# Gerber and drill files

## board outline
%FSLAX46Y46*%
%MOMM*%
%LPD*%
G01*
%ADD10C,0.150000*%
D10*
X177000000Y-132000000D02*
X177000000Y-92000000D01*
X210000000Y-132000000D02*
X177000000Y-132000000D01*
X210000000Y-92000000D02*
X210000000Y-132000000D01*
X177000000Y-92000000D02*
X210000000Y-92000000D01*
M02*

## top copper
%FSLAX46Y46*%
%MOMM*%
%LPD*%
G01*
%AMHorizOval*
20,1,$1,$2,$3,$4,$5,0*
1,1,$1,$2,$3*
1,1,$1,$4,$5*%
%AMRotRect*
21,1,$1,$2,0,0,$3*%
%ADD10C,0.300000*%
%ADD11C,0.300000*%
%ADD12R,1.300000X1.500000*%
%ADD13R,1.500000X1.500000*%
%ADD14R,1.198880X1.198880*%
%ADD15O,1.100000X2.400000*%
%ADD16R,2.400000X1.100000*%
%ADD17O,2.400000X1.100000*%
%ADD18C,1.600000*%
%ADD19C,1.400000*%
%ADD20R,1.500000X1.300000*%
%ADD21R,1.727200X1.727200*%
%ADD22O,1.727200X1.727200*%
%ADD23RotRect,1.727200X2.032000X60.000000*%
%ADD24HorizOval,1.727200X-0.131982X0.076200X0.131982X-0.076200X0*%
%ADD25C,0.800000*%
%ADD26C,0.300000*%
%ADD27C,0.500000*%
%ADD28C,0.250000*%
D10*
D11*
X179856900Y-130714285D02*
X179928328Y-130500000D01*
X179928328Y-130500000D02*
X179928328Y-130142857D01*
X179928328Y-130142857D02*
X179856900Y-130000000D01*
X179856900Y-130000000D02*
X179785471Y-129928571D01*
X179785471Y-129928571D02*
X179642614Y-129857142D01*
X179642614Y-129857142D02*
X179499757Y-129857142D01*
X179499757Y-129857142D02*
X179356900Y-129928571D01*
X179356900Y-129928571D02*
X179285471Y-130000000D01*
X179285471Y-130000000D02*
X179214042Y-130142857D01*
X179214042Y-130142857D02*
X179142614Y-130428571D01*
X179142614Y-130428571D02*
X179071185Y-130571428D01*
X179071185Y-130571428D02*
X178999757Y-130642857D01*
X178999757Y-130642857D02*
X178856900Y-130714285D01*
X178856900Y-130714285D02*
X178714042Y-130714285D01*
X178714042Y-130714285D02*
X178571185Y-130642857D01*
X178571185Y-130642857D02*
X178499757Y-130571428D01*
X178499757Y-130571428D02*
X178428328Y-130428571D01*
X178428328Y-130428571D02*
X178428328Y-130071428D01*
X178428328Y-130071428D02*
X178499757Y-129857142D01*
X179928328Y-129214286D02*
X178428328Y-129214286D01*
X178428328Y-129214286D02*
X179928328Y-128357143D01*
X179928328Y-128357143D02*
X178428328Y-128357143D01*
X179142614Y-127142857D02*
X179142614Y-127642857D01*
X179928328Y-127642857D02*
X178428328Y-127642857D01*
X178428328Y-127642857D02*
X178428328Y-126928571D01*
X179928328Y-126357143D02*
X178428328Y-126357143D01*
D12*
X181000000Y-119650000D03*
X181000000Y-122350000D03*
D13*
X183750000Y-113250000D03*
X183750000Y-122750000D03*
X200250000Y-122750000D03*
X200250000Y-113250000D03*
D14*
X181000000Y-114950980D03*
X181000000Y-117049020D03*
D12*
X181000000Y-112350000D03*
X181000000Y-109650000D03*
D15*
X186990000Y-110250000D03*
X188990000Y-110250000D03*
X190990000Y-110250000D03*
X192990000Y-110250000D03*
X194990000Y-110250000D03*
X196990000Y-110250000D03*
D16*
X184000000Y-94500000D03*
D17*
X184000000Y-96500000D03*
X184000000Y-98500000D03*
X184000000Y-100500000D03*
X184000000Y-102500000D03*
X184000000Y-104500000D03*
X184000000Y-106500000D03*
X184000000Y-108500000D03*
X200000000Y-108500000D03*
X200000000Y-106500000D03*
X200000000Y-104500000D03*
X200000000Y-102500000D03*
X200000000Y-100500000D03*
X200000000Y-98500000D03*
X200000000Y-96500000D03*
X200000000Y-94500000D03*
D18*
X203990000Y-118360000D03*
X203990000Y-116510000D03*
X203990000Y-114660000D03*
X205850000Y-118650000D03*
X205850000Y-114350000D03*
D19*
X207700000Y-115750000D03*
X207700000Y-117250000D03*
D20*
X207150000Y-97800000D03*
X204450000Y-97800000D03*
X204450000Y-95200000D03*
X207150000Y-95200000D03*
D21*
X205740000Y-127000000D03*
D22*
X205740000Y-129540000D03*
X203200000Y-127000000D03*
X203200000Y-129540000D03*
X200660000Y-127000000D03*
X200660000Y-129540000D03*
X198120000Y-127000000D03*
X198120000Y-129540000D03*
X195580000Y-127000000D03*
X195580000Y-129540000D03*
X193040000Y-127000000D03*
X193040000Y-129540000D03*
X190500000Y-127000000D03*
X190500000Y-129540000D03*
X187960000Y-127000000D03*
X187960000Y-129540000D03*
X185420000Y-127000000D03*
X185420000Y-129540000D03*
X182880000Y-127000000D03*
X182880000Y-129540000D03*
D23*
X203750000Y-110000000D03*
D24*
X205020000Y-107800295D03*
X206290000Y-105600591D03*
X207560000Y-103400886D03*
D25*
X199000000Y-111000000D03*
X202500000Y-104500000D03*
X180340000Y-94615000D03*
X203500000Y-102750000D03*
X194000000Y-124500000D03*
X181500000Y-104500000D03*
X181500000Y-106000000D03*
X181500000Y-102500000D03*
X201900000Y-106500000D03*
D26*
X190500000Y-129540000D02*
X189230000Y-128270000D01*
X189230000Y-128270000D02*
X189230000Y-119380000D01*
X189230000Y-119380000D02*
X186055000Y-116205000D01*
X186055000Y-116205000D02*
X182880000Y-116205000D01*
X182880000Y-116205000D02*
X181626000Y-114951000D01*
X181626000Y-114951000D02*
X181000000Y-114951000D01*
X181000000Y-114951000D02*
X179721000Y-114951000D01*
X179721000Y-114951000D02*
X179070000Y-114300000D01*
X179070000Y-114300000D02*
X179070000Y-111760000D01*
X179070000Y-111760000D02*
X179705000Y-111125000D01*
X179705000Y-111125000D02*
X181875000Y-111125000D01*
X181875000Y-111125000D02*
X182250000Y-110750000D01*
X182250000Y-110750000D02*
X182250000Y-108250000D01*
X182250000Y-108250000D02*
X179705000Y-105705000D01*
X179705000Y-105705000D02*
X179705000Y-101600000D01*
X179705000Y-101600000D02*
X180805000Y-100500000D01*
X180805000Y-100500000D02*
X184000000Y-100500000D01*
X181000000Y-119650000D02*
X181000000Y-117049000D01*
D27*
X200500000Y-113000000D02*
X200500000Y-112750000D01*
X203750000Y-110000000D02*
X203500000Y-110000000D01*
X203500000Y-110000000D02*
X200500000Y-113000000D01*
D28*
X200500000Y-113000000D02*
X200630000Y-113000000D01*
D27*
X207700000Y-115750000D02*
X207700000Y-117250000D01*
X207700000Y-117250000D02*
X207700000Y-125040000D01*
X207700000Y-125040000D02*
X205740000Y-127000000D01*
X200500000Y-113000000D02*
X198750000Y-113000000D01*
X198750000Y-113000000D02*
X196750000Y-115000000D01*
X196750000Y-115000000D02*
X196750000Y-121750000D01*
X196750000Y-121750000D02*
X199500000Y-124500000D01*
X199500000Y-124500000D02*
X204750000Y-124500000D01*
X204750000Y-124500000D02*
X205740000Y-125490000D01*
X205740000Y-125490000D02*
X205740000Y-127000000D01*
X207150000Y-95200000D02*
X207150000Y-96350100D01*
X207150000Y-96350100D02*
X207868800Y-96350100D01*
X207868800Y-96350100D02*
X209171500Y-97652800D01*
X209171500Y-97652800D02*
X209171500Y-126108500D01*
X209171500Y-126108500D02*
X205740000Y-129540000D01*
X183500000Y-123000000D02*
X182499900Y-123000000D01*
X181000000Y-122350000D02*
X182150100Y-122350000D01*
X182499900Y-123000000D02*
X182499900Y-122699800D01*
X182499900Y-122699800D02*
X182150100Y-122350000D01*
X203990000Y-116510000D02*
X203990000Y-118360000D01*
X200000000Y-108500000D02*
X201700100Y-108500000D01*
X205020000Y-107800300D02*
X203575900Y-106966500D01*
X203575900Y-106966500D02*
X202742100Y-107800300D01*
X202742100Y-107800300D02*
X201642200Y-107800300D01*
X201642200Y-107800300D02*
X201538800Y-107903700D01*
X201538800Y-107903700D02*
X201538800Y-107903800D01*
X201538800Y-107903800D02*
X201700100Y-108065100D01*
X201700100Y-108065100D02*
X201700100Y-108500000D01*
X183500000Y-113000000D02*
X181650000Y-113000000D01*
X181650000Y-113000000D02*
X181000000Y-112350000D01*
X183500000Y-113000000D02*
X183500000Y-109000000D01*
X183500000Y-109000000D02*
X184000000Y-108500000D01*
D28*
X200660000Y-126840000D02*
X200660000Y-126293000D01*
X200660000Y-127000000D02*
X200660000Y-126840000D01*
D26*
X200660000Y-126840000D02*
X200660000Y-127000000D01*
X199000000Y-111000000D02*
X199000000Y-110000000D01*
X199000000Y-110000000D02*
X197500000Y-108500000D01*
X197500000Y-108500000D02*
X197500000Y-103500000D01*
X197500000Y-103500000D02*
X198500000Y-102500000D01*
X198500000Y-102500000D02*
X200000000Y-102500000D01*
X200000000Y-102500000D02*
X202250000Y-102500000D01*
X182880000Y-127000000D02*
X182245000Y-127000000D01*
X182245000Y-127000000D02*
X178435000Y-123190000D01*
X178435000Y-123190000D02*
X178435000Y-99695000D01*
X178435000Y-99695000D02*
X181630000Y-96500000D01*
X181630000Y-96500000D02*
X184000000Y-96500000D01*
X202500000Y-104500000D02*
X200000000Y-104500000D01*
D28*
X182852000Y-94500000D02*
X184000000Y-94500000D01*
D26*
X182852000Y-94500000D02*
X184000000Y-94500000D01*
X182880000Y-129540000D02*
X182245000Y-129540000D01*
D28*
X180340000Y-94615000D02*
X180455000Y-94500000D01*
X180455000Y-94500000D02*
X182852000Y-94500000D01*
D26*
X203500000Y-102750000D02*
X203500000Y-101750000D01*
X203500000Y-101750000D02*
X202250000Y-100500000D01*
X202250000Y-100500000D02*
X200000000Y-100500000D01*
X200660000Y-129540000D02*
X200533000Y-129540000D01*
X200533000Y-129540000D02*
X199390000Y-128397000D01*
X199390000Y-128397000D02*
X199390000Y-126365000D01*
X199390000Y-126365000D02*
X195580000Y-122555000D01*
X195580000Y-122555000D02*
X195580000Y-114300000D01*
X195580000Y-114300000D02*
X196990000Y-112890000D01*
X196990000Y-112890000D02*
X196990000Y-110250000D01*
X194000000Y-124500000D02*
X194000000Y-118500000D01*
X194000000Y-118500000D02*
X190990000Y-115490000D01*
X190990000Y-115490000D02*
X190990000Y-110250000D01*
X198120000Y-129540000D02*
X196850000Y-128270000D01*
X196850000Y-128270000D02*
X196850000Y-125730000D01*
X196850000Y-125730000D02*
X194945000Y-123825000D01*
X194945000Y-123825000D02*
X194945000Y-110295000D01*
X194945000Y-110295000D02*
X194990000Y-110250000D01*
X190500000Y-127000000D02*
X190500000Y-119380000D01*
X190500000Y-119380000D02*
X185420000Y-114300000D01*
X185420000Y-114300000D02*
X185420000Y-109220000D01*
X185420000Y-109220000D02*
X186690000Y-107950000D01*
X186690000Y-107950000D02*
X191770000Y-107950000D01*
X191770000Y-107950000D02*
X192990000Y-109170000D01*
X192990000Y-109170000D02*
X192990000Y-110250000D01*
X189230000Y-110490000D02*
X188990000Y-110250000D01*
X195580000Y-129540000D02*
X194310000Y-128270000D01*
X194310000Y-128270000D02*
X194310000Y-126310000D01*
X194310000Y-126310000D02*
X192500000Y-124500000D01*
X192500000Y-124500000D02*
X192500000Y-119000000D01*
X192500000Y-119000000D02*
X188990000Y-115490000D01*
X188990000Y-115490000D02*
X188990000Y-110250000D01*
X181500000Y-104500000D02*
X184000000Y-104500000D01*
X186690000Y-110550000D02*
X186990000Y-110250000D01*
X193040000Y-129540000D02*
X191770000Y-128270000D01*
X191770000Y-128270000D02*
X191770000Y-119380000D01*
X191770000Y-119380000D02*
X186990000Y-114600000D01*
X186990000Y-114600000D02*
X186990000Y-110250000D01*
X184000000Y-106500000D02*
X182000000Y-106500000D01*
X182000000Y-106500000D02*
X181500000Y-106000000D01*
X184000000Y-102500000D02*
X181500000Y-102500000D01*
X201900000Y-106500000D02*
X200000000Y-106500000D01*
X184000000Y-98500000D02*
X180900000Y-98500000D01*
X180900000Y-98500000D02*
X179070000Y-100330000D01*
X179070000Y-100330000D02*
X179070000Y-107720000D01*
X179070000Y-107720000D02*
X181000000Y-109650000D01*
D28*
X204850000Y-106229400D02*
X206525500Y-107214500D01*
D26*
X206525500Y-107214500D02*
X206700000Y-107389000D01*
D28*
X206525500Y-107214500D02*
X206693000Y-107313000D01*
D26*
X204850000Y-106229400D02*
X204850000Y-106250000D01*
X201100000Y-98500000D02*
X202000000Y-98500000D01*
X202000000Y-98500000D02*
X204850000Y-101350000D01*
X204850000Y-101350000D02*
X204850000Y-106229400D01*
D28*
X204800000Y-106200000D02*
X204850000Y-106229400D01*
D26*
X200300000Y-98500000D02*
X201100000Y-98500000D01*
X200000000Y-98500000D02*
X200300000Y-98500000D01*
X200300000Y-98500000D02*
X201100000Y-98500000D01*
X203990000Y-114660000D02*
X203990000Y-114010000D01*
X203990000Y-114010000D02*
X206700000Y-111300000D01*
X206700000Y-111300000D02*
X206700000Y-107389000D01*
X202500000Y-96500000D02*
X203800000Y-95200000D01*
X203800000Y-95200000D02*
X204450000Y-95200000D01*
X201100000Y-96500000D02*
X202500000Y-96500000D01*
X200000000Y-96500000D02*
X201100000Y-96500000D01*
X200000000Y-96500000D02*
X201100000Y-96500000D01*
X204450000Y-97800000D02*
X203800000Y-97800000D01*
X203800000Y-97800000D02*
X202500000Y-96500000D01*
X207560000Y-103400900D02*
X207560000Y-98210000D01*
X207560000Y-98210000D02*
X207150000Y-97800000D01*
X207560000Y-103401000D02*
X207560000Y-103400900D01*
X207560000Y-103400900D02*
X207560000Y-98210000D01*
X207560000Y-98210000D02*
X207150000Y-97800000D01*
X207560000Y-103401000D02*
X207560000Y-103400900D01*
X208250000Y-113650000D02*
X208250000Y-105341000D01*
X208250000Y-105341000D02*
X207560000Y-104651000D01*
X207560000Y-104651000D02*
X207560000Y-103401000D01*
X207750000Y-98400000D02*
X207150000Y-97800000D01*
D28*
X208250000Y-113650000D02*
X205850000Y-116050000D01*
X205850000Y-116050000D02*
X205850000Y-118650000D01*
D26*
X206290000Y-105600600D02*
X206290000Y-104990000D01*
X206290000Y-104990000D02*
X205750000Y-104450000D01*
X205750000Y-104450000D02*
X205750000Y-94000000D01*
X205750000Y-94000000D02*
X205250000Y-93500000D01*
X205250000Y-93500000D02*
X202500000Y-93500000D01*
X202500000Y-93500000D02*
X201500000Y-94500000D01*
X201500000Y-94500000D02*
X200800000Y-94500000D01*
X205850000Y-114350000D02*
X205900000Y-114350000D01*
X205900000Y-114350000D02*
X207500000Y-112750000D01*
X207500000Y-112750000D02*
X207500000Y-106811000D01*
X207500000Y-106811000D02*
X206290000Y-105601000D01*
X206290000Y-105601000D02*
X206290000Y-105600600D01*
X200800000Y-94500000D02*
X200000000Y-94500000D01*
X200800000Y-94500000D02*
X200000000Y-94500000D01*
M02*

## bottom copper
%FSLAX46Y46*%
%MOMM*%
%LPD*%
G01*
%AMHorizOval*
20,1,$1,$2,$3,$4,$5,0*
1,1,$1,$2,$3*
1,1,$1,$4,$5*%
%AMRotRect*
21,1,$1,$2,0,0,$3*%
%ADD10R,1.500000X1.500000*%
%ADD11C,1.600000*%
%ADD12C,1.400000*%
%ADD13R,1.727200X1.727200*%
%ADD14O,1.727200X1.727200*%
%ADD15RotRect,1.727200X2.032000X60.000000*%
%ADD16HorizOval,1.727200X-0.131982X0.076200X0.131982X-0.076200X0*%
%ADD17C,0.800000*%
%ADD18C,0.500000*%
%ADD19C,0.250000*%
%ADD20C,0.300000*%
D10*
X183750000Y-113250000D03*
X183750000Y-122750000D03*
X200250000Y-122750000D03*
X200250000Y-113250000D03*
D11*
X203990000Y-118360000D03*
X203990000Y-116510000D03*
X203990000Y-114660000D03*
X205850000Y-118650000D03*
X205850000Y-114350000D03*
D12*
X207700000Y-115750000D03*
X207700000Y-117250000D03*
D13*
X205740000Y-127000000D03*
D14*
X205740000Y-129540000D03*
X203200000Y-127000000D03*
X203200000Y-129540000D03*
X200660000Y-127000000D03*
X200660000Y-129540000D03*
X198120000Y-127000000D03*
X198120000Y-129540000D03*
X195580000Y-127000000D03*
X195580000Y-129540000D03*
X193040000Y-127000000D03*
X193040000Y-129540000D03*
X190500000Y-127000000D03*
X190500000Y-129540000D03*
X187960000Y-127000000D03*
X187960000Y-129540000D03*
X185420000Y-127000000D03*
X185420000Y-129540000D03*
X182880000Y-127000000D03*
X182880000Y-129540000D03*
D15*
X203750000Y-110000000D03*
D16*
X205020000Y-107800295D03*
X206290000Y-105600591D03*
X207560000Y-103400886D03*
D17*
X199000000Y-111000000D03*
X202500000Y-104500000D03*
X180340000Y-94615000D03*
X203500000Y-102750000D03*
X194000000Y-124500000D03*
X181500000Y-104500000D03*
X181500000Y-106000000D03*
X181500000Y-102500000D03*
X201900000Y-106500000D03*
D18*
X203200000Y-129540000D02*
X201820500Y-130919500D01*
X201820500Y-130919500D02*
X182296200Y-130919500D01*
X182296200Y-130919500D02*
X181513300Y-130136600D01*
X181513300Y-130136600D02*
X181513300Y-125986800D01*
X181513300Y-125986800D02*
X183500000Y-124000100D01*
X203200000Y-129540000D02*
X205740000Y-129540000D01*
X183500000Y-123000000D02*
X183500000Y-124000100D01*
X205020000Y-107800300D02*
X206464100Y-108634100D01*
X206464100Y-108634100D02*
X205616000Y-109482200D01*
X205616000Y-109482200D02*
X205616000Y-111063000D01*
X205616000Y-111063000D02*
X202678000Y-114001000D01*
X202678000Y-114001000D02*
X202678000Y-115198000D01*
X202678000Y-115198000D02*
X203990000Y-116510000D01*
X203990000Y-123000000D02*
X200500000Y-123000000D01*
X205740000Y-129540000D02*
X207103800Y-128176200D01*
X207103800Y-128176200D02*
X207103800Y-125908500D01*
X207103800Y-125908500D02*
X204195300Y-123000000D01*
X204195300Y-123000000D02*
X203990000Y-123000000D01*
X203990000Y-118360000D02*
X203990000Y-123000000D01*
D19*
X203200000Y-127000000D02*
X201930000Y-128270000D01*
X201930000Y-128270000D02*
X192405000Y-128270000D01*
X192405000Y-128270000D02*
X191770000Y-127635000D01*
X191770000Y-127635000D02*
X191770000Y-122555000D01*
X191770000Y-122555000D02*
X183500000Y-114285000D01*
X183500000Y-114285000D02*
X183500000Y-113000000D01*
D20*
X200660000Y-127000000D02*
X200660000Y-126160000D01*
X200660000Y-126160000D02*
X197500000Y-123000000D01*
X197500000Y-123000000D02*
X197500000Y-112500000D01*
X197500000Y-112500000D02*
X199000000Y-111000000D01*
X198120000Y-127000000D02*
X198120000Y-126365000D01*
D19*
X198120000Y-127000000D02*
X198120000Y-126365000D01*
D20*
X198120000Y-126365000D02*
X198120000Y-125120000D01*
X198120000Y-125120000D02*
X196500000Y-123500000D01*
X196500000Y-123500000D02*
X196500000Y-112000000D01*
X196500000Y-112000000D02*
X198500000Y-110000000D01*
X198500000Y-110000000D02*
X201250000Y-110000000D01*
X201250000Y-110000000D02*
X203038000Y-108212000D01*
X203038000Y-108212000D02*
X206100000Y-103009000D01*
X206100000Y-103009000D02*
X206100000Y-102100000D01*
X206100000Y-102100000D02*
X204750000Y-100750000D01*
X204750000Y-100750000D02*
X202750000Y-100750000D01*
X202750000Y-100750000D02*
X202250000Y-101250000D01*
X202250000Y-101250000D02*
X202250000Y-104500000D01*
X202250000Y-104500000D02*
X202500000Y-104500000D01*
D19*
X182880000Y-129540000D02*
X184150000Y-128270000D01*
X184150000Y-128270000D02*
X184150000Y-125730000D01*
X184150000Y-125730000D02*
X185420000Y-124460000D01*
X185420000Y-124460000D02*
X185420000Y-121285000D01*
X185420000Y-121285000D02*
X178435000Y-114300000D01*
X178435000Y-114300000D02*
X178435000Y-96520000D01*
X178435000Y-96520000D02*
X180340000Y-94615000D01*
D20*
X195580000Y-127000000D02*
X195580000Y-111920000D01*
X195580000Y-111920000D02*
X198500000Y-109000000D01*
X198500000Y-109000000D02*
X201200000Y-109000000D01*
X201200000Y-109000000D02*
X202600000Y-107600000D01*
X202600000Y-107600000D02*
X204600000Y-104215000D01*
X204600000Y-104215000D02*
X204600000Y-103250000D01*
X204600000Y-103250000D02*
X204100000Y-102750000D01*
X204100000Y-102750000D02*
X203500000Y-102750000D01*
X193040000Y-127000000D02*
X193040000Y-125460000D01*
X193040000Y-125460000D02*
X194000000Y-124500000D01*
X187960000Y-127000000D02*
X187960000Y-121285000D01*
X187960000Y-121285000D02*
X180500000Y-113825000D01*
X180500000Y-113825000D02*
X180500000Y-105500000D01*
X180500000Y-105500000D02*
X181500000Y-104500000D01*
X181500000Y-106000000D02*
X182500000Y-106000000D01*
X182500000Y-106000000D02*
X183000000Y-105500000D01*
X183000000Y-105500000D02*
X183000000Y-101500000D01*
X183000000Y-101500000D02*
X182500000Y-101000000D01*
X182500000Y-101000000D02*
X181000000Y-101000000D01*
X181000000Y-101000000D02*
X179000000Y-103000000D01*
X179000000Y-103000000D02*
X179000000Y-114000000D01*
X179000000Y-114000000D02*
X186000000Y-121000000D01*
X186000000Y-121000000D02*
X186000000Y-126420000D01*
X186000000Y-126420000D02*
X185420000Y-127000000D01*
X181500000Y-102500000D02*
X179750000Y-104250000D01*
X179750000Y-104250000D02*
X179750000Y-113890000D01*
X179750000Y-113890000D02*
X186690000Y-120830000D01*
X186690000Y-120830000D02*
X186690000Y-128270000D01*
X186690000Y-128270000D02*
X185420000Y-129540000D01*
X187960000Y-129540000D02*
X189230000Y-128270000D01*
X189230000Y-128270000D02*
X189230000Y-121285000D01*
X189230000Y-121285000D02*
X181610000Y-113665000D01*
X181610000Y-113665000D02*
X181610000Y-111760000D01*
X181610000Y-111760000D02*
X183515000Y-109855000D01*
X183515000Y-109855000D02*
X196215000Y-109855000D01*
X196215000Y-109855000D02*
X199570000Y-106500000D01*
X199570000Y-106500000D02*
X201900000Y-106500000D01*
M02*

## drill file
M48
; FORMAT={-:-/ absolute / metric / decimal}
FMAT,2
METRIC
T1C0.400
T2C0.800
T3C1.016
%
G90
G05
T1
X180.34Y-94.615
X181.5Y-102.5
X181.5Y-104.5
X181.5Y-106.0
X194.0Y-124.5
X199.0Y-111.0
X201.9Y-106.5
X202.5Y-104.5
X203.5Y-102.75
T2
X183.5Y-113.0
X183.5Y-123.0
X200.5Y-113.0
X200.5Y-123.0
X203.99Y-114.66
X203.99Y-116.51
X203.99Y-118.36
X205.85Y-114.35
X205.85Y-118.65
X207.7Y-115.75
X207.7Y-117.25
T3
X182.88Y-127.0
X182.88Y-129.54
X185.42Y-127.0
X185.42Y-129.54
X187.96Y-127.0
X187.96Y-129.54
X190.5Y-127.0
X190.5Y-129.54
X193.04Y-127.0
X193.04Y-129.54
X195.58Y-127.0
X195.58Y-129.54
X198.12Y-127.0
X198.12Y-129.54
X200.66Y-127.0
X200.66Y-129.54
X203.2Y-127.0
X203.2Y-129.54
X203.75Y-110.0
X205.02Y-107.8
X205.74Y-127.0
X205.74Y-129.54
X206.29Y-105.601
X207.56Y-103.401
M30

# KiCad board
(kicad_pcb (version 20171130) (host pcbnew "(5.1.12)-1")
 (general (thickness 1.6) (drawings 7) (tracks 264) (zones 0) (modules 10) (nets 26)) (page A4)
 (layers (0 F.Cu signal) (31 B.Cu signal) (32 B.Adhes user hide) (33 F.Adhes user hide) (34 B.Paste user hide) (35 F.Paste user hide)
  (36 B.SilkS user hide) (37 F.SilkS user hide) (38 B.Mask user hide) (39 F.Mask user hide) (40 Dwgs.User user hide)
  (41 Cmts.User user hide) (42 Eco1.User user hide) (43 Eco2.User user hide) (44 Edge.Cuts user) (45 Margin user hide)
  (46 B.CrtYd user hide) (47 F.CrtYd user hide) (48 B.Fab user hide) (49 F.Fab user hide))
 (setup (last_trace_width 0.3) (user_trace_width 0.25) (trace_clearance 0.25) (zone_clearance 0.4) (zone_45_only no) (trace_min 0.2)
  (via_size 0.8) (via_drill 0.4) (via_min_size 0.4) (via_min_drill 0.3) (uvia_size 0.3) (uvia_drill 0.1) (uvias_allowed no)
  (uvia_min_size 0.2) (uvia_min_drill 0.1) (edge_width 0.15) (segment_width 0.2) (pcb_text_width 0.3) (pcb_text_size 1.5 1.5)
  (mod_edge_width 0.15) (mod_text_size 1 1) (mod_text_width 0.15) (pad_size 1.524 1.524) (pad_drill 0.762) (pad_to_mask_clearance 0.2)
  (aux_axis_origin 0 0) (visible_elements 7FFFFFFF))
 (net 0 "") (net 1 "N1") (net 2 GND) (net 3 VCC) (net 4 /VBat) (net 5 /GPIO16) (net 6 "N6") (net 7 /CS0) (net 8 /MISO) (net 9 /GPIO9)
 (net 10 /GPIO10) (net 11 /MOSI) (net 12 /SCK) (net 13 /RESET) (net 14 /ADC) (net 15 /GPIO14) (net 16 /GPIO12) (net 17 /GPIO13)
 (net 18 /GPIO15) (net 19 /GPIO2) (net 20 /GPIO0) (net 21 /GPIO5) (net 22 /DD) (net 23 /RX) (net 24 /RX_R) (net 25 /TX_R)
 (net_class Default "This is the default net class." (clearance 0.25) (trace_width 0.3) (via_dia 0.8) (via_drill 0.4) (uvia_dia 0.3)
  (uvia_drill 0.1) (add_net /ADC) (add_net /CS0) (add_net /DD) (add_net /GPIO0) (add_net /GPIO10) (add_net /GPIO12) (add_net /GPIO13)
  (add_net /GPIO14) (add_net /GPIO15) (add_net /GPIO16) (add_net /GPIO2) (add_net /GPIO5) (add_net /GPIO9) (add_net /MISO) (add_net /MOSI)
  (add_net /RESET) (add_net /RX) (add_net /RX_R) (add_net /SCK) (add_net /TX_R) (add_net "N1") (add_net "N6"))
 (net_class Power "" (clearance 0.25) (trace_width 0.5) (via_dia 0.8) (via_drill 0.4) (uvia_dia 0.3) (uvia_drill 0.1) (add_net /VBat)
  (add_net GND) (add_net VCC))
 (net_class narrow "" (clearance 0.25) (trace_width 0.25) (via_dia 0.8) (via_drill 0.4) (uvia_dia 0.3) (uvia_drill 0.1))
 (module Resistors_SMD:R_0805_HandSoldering (layer F.Cu) (at 181 121 270)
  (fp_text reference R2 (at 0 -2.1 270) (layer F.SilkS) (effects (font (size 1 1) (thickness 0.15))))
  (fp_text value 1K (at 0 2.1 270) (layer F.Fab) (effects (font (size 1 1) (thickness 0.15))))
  (pad 1 smd rect (at -1.35 0 270) (size 1.5 1.3) (layers F.Cu F.Paste F.Mask) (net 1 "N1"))
  (pad 2 smd rect (at 1.35 0 270) (size 1.5 1.3) (layers F.Cu F.Paste F.Mask) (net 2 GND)))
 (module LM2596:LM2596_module (layer F.Cu) (at 192 118)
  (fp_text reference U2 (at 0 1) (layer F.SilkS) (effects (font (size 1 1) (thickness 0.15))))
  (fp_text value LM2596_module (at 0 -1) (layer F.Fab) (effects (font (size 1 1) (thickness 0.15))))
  (pad 1 thru_hole rect (at -8.5 -5) (size 1.5 1.5) (drill 0.8 (offset 0.25 0.25)) (layers *.Cu *.Mask F.SilkS) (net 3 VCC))
  (pad 2 thru_hole rect (at -8.5 5) (size 1.5 1.5) (drill 0.8 (offset 0.25 -0.25)) (layers *.Cu *.Mask F.SilkS) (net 2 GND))
  (pad 3 thru_hole rect (at 8.5 5) (size 1.5 1.5) (drill 0.8 (offset -0.25 -0.25)) (layers *.Cu *.Mask F.SilkS) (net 2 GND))
  (pad 4 thru_hole rect (at 8.5 -5) (size 1.5 1.5) (drill 0.8 (offset -0.25 0.25)) (layers *.Cu *.Mask F.SilkS) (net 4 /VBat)))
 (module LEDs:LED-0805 (layer F.Cu) (at 181 116 90)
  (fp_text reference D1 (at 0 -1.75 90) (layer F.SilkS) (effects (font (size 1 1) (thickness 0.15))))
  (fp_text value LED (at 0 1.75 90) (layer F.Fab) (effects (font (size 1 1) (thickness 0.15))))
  (pad 2 smd rect (at 1.04902 0 270) (size 1.19888 1.19888) (layers F.Cu F.Paste F.Mask) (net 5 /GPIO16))
  (pad 1 smd rect (at -1.04902 0 270) (size 1.19888 1.19888) (layers F.Cu F.Paste F.Mask) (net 1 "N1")))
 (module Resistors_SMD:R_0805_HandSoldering (layer F.Cu) (at 181 111 90)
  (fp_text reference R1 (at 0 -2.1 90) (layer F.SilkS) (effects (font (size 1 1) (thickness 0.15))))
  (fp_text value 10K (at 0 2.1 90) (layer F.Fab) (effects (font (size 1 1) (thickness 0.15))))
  (pad 1 smd rect (at -1.35 0 90) (size 1.5 1.3) (layers F.Cu F.Paste F.Mask) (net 3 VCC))
  (pad 2 smd rect (at 1.35 0 90) (size 1.5 1.3) (layers F.Cu F.Paste F.Mask) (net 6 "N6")))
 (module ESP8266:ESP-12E (layer F.Cu) (at 184 94.5)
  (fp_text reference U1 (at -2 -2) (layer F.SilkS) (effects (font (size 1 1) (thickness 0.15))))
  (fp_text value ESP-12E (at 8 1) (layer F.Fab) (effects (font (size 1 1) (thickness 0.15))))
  (pad 9 smd oval (at 2.99 15.75 90) (size 2.4 1.1) (layers F.Cu F.Paste F.Mask) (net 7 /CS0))
  (pad 10 smd oval (at 4.99 15.75 90) (size 2.4 1.1) (layers F.Cu F.Paste F.Mask) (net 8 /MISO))
  (pad 11 smd oval (at 6.99 15.75 90) (size 2.4 1.1) (layers F.Cu F.Paste F.Mask) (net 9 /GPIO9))
  (pad 12 smd oval (at 8.99 15.75 90) (size 2.4 1.1) (layers F.Cu F.Paste F.Mask) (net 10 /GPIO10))
  (pad 13 smd oval (at 10.99 15.75 90) (size 2.4 1.1) (layers F.Cu F.Paste F.Mask) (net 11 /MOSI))
  (pad 14 smd oval (at 12.99 15.75 90) (size 2.4 1.1) (layers F.Cu F.Paste F.Mask) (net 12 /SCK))
  (pad 1 smd rect (at 0 0) (size 2.4 1.1) (layers F.Cu F.Paste F.Mask) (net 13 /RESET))
  (pad 2 smd oval (at 0 2) (size 2.4 1.1) (layers F.Cu F.Paste F.Mask) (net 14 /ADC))
  (pad 3 smd oval (at 0 4) (size 2.4 1.1) (layers F.Cu F.Paste F.Mask) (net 6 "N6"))
  (pad 4 smd oval (at 0 6) (size 2.4 1.1) (layers F.Cu F.Paste F.Mask) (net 5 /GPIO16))
  (pad 5 smd oval (at 0 8) (size 2.4 1.1) (layers F.Cu F.Paste F.Mask) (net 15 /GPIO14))
  (pad 6 smd oval (at 0 10) (size 2.4 1.1) (layers F.Cu F.Paste F.Mask) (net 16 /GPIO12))
  (pad 7 smd oval (at 0 12) (size 2.4 1.1) (layers F.Cu F.Paste F.Mask) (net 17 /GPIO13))
  (pad 8 smd oval (at 0 14) (size 2.4 1.1) (layers F.Cu F.Paste F.Mask) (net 3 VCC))
  (pad 15 smd oval (at 16 14) (size 2.4 1.1) (layers F.Cu F.Paste F.Mask) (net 2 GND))
  (pad 16 smd oval (at 16 12) (size 2.4 1.1) (layers F.Cu F.Paste F.Mask) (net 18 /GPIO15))
  (pad 17 smd oval (at 16 10) (size 2.4 1.1) (layers F.Cu F.Paste F.Mask) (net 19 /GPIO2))
  (pad 18 smd oval (at 16 8) (size 2.4 1.1) (layers F.Cu F.Paste F.Mask) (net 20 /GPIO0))
  (pad 19 smd oval (at 16 6) (size 2.4 1.1) (layers F.Cu F.Paste F.Mask) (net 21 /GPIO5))
  (pad 20 smd oval (at 16 4) (size 2.4 1.1) (layers F.Cu F.Paste F.Mask) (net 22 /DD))
  (pad 21 smd oval (at 16 2) (size 2.4 1.1) (layers F.Cu F.Paste F.Mask) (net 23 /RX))
  (pad 22 smd oval (at 16 0) (size 2.4 1.1) (layers F.Cu F.Paste F.Mask) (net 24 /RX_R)))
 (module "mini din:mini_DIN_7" (layer F.Cu) (at 213.5 116.5 90)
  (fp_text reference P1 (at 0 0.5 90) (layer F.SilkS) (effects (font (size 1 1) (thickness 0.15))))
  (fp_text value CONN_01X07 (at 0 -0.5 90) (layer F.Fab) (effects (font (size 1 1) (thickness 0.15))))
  (pad 7 thru_hole circle (at -1.86 -9.51 90) (size 1.6 1.6) (drill 0.8) (layers *.Cu *.Mask F.SilkS) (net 2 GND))
  (pad 6 thru_hole circle (at -0.01 -9.51 90) (size 1.6 1.6) (drill 0.8) (layers *.Cu *.Mask F.SilkS) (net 2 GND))
  (pad 5 thru_hole circle (at 1.84 -9.51 90) (size 1.6 1.6) (drill 0.8) (layers *.Cu *.Mask F.SilkS) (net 22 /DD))
  (pad 4 thru_hole circle (at -2.15 -7.65 90) (size 1.6 1.6) (drill 0.8) (layers *.Cu *.Mask F.SilkS) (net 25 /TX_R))
  (pad 3 thru_hole circle (at 2.15 -7.65 90) (size 1.6 1.6) (drill 0.8) (layers *.Cu *.Mask F.SilkS) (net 24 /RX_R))
  (pad 1 thru_hole circle (at 0.75 -5.8 90) (size 1.4 1.4) (drill 0.8) (layers *.Cu *.Mask F.SilkS) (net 4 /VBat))
  (pad 2 thru_hole circle (at -0.75 -5.8 90) (size 1.4 1.4) (drill 0.8) (layers *.Cu *.Mask F.SilkS) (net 4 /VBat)))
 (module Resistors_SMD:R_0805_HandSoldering (layer F.Cu) (at 205.8 97.8 180)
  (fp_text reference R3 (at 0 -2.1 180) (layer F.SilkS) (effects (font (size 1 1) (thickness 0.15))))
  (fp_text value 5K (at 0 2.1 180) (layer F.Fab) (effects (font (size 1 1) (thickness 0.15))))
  (pad 1 smd rect (at -1.35 0 180) (size 1.5 1.3) (layers F.Cu F.Paste F.Mask) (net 25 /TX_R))
  (pad 2 smd rect (at 1.35 0 180) (size 1.5 1.3) (layers F.Cu F.Paste F.Mask) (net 23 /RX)))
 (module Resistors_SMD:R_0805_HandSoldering (layer F.Cu) (at 205.8 95.2)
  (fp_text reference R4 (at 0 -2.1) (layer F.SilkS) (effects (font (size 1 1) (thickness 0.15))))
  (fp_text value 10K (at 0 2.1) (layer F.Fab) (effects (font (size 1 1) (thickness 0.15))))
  (pad 1 smd rect (at -1.35 0) (size 1.5 1.3) (layers F.Cu F.Paste F.Mask) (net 23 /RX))
  (pad 2 smd rect (at 1.35 0) (size 1.5 1.3) (layers F.Cu F.Paste F.Mask) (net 2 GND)))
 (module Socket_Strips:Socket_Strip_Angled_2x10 (layer B.Cu) (at 205.74 127 180)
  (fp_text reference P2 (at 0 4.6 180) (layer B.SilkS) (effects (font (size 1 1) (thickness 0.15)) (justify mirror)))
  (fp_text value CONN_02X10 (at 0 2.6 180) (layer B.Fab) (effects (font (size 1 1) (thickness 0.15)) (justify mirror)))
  (pad 1 thru_hole rect (at 0 0 180) (size 1.7272 1.7272) (drill 1.016) (layers *.Cu *.Mask B.SilkS) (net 4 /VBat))
  (pad 2 thru_hole oval (at 0 -2.54 180) (size 1.7272 1.7272) (drill 1.016) (layers *.Cu *.Mask B.SilkS) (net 2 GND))
  (pad 3 thru_hole oval (at 2.54 0 180) (size 1.7272 1.7272) (drill 1.016) (layers *.Cu *.Mask B.SilkS) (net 3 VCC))
  (pad 4 thru_hole oval (at 2.54 -2.54 180) (size 1.7272 1.7272) (drill 1.016) (layers *.Cu *.Mask B.SilkS) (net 2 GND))
  (pad 5 thru_hole oval (at 5.08 0 180) (size 1.7272 1.7272) (drill 1.016) (layers *.Cu *.Mask B.SilkS) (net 20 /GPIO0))
  (pad 6 thru_hole oval (at 5.08 -2.54 180) (size 1.7272 1.7272) (drill 1.016) (layers *.Cu *.Mask B.SilkS) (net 12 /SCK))
  (pad 7 thru_hole oval (at 7.62 0 180) (size 1.7272 1.7272) (drill 1.016) (layers *.Cu *.Mask B.SilkS) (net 19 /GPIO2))
  (pad 8 thru_hole oval (at 7.62 -2.54 180) (size 1.7272 1.7272) (drill 1.016) (layers *.Cu *.Mask B.SilkS) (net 11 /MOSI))
  (pad 9 thru_hole oval (at 10.16 0 180) (size 1.7272 1.7272) (drill 1.016) (layers *.Cu *.Mask B.SilkS) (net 21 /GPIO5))
  (pad 10 thru_hole oval (at 10.16 -2.54 180) (size 1.7272 1.7272) (drill 1.016) (layers *.Cu *.Mask B.SilkS) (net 8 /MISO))
  (pad 11 thru_hole oval (at 12.7 0 180) (size 1.7272 1.7272) (drill 1.016) (layers *.Cu *.Mask B.SilkS) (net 9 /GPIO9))
  (pad 12 thru_hole oval (at 12.7 -2.54 180) (size 1.7272 1.7272) (drill 1.016) (layers *.Cu *.Mask B.SilkS) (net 7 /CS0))
  (pad 13 thru_hole oval (at 15.24 0 180) (size 1.7272 1.7272) (drill 1.016) (layers *.Cu *.Mask B.SilkS) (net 10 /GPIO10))
  (pad 14 thru_hole oval (at 15.24 -2.54 180) (size 1.7272 1.7272) (drill 1.016) (layers *.Cu *.Mask B.SilkS) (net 5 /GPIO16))
  (pad 15 thru_hole oval (at 17.78 0 180) (size 1.7272 1.7272) (drill 1.016) (layers *.Cu *.Mask B.SilkS) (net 16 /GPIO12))
  (pad 16 thru_hole oval (at 17.78 -2.54 180) (size 1.7272 1.7272) (drill 1.016) (layers *.Cu *.Mask B.SilkS) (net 18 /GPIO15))
  (pad 17 thru_hole oval (at 20.32 0 180) (size 1.7272 1.7272) (drill 1.016) (layers *.Cu *.Mask B.SilkS) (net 17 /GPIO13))
  (pad 18 thru_hole oval (at 20.32 -2.54 180) (size 1.7272 1.7272) (drill 1.016) (layers *.Cu *.Mask B.SilkS) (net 15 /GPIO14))
  (pad 19 thru_hole oval (at 22.86 0 180) (size 1.7272 1.7272) (drill 1.016) (layers *.Cu *.Mask B.SilkS) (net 14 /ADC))
  (pad 20 thru_hole oval (at 22.86 -2.54 180) (size 1.7272 1.7272) (drill 1.016) (layers *.Cu *.Mask B.SilkS) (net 13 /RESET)))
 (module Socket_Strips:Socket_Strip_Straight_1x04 (layer F.Cu) (at 203.75 110 60)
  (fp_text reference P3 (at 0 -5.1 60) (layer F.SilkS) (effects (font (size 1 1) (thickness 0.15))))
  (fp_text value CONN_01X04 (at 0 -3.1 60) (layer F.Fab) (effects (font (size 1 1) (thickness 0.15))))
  (pad 1 thru_hole rect (at 0 0 60) (size 1.7272 2.032) (drill 1.016) (layers *.Cu *.Mask F.SilkS) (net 4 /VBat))
  (pad 2 thru_hole oval (at 2.54 0 60) (size 1.7272 2.032) (drill 1.016) (layers *.Cu *.Mask F.SilkS) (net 2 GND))
  (pad 3 thru_hole oval (at 5.08 0 60) (size 1.7272 2.032) (drill 1.016) (layers *.Cu *.Mask F.SilkS) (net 24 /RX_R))
  (pad 4 thru_hole oval (at 7.62 0 60) (size 1.7272 2.032) (drill 1.016) (layers *.Cu *.Mask F.SilkS) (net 25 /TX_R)))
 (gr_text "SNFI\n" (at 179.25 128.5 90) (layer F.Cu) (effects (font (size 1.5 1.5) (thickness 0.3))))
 (gr_line (start 177 132) (end 177 92) (angle 90) (layer Edge.Cuts) (width 0.15))
 (gr_line (start 210 132) (end 177 132) (angle 90) (layer Edge.Cuts) (width 0.15))
 (gr_line (start 210 92) (end 210 132) (angle 90) (layer Edge.Cuts) (width 0.15))
 (gr_line (start 177 92) (end 210 92) (angle 90) (layer Edge.Cuts) (width 0.15))
 (segment (start 190.5 129.54) (end 189.23 128.27) (width 0.3) (layer F.Cu) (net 5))
 (segment (start 189.23 128.27) (end 189.23 119.38) (width 0.3) (layer F.Cu) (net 5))
 (segment (start 189.23 119.38) (end 186.055 116.205) (width 0.3) (layer F.Cu) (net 5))
 (segment (start 186.055 116.205) (end 182.88 116.205) (width 0.3) (layer F.Cu) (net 5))
 (segment (start 182.88 116.205) (end 181.626 114.951) (width 0.3) (layer F.Cu) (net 5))
 (segment (start 181.626 114.951) (end 181 114.951) (width 0.3) (layer F.Cu) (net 5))
 (segment (start 181 114.951) (end 179.721 114.951) (width 0.3) (layer F.Cu) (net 5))
 (segment (start 179.721 114.951) (end 179.07 114.3) (width 0.3) (layer F.Cu) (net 5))
 (segment (start 179.07 114.3) (end 179.07 111.76) (width 0.3) (layer F.Cu) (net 5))
 (segment (start 179.07 111.76) (end 179.705 111.125) (width 0.3) (layer F.Cu) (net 5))
 (segment (start 179.705 111.125) (end 181.875 111.125) (width 0.3) (layer F.Cu) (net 5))
 (segment (start 181.875 111.125) (end 182.25 110.75) (width 0.3) (layer F.Cu) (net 5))
 (segment (start 182.25 110.75) (end 182.25 108.25) (width 0.3) (layer F.Cu) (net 5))
 (segment (start 182.25 108.25) (end 179.705 105.705) (width 0.3) (layer F.Cu) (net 5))
 (segment (start 179.705 105.705) (end 179.705 101.6) (width 0.3) (layer F.Cu) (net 5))
 (segment (start 179.705 101.6) (end 180.805 100.5) (width 0.3) (layer F.Cu) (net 5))
 (segment (start 180.805 100.5) (end 184 100.5) (width 0.3) (layer F.Cu) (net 5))
 (segment (start 181 119.65) (end 181 117.049) (width 0.3) (layer F.Cu) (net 1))
 (segment (start 200.5 113) (end 200.5 112.75) (width 0.5) (layer F.Cu) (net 4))
 (segment (start 203.75 110) (end 203.5 110) (width 0.5) (layer F.Cu) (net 4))
 (segment (start 203.5 110) (end 200.5 113) (width 0.5) (layer F.Cu) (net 4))
 (segment (start 200.5 113) (end 200.63 113) (width 0.25) (layer F.Cu) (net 4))
 (segment (start 207.7 115.75) (end 207.7 117.25) (width 0.5) (layer F.Cu) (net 4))
 (segment (start 207.7 117.25) (end 207.7 125.04) (width 0.5) (layer F.Cu) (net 4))
 (segment (start 207.7 125.04) (end 205.74 127) (width 0.5) (layer F.Cu) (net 4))
 (segment (start 200.5 113) (end 198.75 113) (width 0.5) (layer F.Cu) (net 4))
 (segment (start 198.75 113) (end 196.75 115) (width 0.5) (layer F.Cu) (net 4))
 (segment (start 196.75 115) (end 196.75 121.75) (width 0.5) (layer F.Cu) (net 4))
 (segment (start 196.75 121.75) (end 199.5 124.5) (width 0.5) (layer F.Cu) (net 4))
 (segment (start 199.5 124.5) (end 204.75 124.5) (width 0.5) (layer F.Cu) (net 4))
 (segment (start 204.75 124.5) (end 205.74 125.49) (width 0.5) (layer F.Cu) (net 4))
 (segment (start 205.74 125.49) (end 205.74 127) (width 0.5) (layer F.Cu) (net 4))
 (segment (start 207.15 95.2) (end 207.15 96.3501) (width 0.5) (layer F.Cu) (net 2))
 (segment (start 207.15 96.3501) (end 207.8688 96.3501) (width 0.5) (layer F.Cu) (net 2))
 (segment (start 207.8688 96.3501) (end 209.1715 97.6528) (width 0.5) (layer F.Cu) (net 2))
 (segment (start 209.1715 97.6528) (end 209.1715 126.1085) (width 0.5) (layer F.Cu) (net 2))
 (segment (start 209.1715 126.1085) (end 205.74 129.54) (width 0.5) (layer F.Cu) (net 2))
 (segment (start 183.5 123) (end 182.4999 123) (width 0.5) (layer F.Cu) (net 2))
 (segment (start 181 122.35) (end 182.1501 122.35) (width 0.5) (layer F.Cu) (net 2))
 (segment (start 182.4999 123) (end 182.4999 122.6998) (width 0.5) (layer F.Cu) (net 2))
 (segment (start 182.4999 122.6998) (end 182.1501 122.35) (width 0.5) (layer F.Cu) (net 2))
 (segment (start 203.2 129.54) (end 201.8205 130.9195) (width 0.5) (layer B.Cu) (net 2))
 (segment (start 201.8205 130.9195) (end 182.2962 130.9195) (width 0.5) (layer B.Cu) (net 2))
 (segment (start 182.2962 130.9195) (end 181.5133 130.1366) (width 0.5) (layer B.Cu) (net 2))
 (segment (start 181.5133 130.1366) (end 181.5133 125.9868) (width 0.5) (layer B.Cu) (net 2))
 (segment (start 181.5133 125.9868) (end 183.5 124.0001) (width 0.5) (layer B.Cu) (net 2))
 (segment (start 203.2 129.54) (end 205.74 129.54) (width 0.5) (layer B.Cu) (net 2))
 (segment (start 183.5 123) (end 183.5 124.0001) (width 0.5) (layer B.Cu) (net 2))
 (segment (start 205.02 107.8003) (end 206.4641 108.6341) (width 0.5) (layer B.Cu) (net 2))
 (segment (start 206.4641 108.6341) (end 205.616 109.4822) (width 0.5) (layer B.Cu) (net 2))
 (segment (start 205.616 109.4822) (end 205.616 111.063) (width 0.5) (layer B.Cu) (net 2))
 (segment (start 205.616 111.063) (end 202.678 114.001) (width 0.5) (layer B.Cu) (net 2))
 (segment (start 202.678 114.001) (end 202.678 115.198) (width 0.5) (layer B.Cu) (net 2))
 (segment (start 202.678 115.198) (end 203.99 116.51) (width 0.5) (layer B.Cu) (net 2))
 (segment (start 203.99 123) (end 200.5 123) (width 0.5) (layer B.Cu) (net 2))
 (segment (start 205.74 129.54) (end 207.1038 128.1762) (width 0.5) (layer B.Cu) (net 2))
 (segment (start 207.1038 128.1762) (end 207.1038 125.9085) (width 0.5) (layer B.Cu) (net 2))
 (segment (start 207.1038 125.9085) (end 204.1953 123) (width 0.5) (layer B.Cu) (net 2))
 (segment (start 204.1953 123) (end 203.99 123) (width 0.5) (layer B.Cu) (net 2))
 (segment (start 203.99 118.36) (end 203.99 123) (width 0.5) (layer B.Cu) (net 2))
 (segment (start 203.99 116.51) (end 203.99 118.36) (width 0.5) (layer F.Cu) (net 2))
 (segment (start 200 108.5) (end 201.7001 108.5) (width 0.5) (layer F.Cu) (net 2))
 (segment (start 205.02 107.8003) (end 203.5759 106.9665) (width 0.5) (layer F.Cu) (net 2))
 (segment (start 203.5759 106.9665) (end 202.7421 107.8003) (width 0.5) (layer F.Cu) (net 2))
 (segment (start 202.7421 107.8003) (end 201.6422 107.8003) (width 0.5) (layer F.Cu) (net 2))
 (segment (start 201.6422 107.8003) (end 201.5388 107.9037) (width 0.5) (layer F.Cu) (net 2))
 (segment (start 201.5388 107.9037) (end 201.5388 107.9038) (width 0.5) (layer F.Cu) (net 2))
 (segment (start 201.5388 107.9038) (end 201.7001 108.0651) (width 0.5) (layer F.Cu) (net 2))
 (segment (start 201.7001 108.0651) (end 201.7001 108.5) (width 0.5) (layer F.Cu) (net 2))
 (segment (start 183.5 113) (end 181.65 113) (width 0.5) (layer F.Cu) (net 3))
 (segment (start 181.65 113) (end 181 112.35) (width 0.5) (layer F.Cu) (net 3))
 (segment (start 183.5 113) (end 183.5 109) (width 0.5) (layer F.Cu) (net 3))
 (segment (start 183.5 109) (end 184 108.5) (width 0.5) (layer F.Cu) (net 3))
 (segment (start 203.2 127) (end 201.93 128.27) (width 0.25) (layer B.Cu) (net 3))
 (segment (start 201.93 128.27) (end 192.405 128.27) (width 0.25) (layer B.Cu) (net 3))
 (segment (start 192.405 128.27) (end 191.77 127.635) (width 0.25) (layer B.Cu) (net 3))
 (segment (start 191.77 127.635) (end 191.77 122.555) (width 0.25) (layer B.Cu) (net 3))
 (segment (start 191.77 122.555) (end 183.5 114.285) (width 0.25) (layer B.Cu) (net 3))
 (segment (start 183.5 114.285) (end 183.5 113) (width 0.25) (layer B.Cu) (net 3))
 (segment (start 200.66 126.84) (end 200.66 126.293) (width 0.25) (layer F.Cu) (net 20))
 (segment (start 200.66 127) (end 200.66 126.84) (width 0.25) (layer F.Cu) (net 20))
 (segment (start 200.66 126.84) (end 200.66 127) (width 0.3) (layer F.Cu) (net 20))
 (segment (start 200.66 127) (end 200.66 126.16) (width 0.3) (layer B.Cu) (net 20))
 (segment (start 200.66 126.16) (end 197.5 123) (width 0.3) (layer B.Cu) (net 20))
 (segment (start 197.5 123) (end 197.5 112.5) (width 0.3) (layer B.Cu) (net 20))
 (segment (start 197.5 112.5) (end 199 111) (width 0.3) (layer B.Cu) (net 20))
 (segment (start 199 111) (end 199 110) (width 0.3) (layer F.Cu) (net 20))
 (segment (start 199 110) (end 197.5 108.5) (width 0.3) (layer F.Cu) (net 20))
 (segment (start 197.5 108.5) (end 197.5 103.5) (width 0.3) (layer F.Cu) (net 20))
 (segment (start 197.5 103.5) (end 198.5 102.5) (width 0.3) (layer F.Cu) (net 20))
 (segment (start 198.5 102.5) (end 200 102.5) (width 0.3) (layer F.Cu) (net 20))
 (segment (start 200 102.5) (end 202.25 102.5) (width 0.3) (layer F.Cu) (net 20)) (via (at 199 111) (size 0.8) (layers F.Cu B.Cu) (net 20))
 (segment (start 182.88 127) (end 182.245 127) (width 0.3) (layer F.Cu) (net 14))
 (segment (start 182.245 127) (end 178.435 123.19) (width 0.3) (layer F.Cu) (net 14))
 (segment (start 178.435 123.19) (end 178.435 99.695) (width 0.3) (layer F.Cu) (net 14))
 (segment (start 178.435 99.695) (end 181.63 96.5) (width 0.3) (layer F.Cu) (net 14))
 (segment (start 181.63 96.5) (end 184 96.5) (width 0.3) (layer F.Cu) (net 14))
 (segment (start 198.12 127) (end 198.12 126.365) (width 0.3) (layer B.Cu) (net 19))
 (segment (start 198.12 127) (end 198.12 126.365) (width 0.25) (layer B.Cu) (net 19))
 (segment (start 198.12 126.365) (end 198.12 125.12) (width 0.3) (layer B.Cu) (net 19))
 (segment (start 198.12 125.12) (end 196.5 123.5) (width 0.3) (layer B.Cu) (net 19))
 (segment (start 196.5 123.5) (end 196.5 112) (width 0.3) (layer B.Cu) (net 19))
 (segment (start 196.5 112) (end 198.5 110) (width 0.3) (layer B.Cu) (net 19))
 (segment (start 198.5 110) (end 201.25 110) (width 0.3) (layer B.Cu) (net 19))
 (segment (start 201.25 110) (end 203.038 108.212) (width 0.3) (layer B.Cu) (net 19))
 (segment (start 203.038 108.212) (end 206.1 103.009) (width 0.3) (layer B.Cu) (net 19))
 (segment (start 206.1 103.009) (end 206.1 102.1) (width 0.3) (layer B.Cu) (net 19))
 (segment (start 206.1 102.1) (end 204.75 100.75) (width 0.3) (layer B.Cu) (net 19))
 (segment (start 204.75 100.75) (end 202.75 100.75) (width 0.3) (layer B.Cu) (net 19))
 (segment (start 202.75 100.75) (end 202.25 101.25) (width 0.3) (layer B.Cu) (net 19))
 (segment (start 202.25 101.25) (end 202.25 104.5) (width 0.3) (layer B.Cu) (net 19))
 (segment (start 202.25 104.5) (end 202.5 104.5) (width 0.3) (layer B.Cu) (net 19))
 (segment (start 202.5 104.5) (end 200 104.5) (width 0.3) (layer F.Cu) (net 19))
 (via (at 202.5 104.5) (size 0.8) (layers F.Cu B.Cu) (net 19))
 (segment (start 182.852 94.5) (end 184 94.5) (width 0.25) (layer F.Cu) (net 13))
 (segment (start 182.852 94.5) (end 184 94.5) (width 0.3) (layer F.Cu) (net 13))
 (segment (start 182.88 129.54) (end 182.245 129.54) (width 0.3) (layer F.Cu) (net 13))
 (segment (start 182.88 129.54) (end 184.15 128.27) (width 0.25) (layer B.Cu) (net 13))
 (segment (start 184.15 128.27) (end 184.15 125.73) (width 0.25) (layer B.Cu) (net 13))
 (segment (start 184.15 125.73) (end 185.42 124.46) (width 0.25) (layer B.Cu) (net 13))
 (segment (start 185.42 124.46) (end 185.42 121.285) (width 0.25) (layer B.Cu) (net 13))
 (segment (start 185.42 121.285) (end 178.435 114.3) (width 0.25) (layer B.Cu) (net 13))
 (segment (start 178.435 114.3) (end 178.435 96.52) (width 0.25) (layer B.Cu) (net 13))
 (segment (start 178.435 96.52) (end 180.34 94.615) (width 0.25) (layer B.Cu) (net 13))
 (segment (start 180.34 94.615) (end 180.455 94.5) (width 0.25) (layer F.Cu) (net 13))
 (segment (start 180.455 94.5) (end 182.852 94.5) (width 0.25) (layer F.Cu) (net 13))
 (via (at 180.34 94.615) (size 0.8) (layers F.Cu B.Cu) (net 13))
 (segment (start 203.5 102.75) (end 203.5 101.75) (width 0.3) (layer F.Cu) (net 21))
 (segment (start 203.5 101.75) (end 202.25 100.5) (width 0.3) (layer F.Cu) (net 21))
 (segment (start 202.25 100.5) (end 200 100.5) (width 0.3) (layer F.Cu) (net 21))
 (segment (start 195.58 127) (end 195.58 111.92) (width 0.3) (layer B.Cu) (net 21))
 (segment (start 195.58 111.92) (end 198.5 109) (width 0.3) (layer B.Cu) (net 21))
 (segment (start 198.5 109) (end 201.2 109) (width 0.3) (layer B.Cu) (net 21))
 (segment (start 201.2 109) (end 202.6 107.6) (width 0.3) (layer B.Cu) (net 21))
 (segment (start 202.6 107.6) (end 204.6 104.215) (width 0.3) (layer B.Cu) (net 21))
 (segment (start 204.6 104.215) (end 204.6 103.25) (width 0.3) (layer B.Cu) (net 21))
 (segment (start 204.6 103.25) (end 204.1 102.75) (width 0.3) (layer B.Cu) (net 21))
 (segment (start 204.1 102.75) (end 203.5 102.75) (width 0.3) (layer B.Cu) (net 21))
 (via (at 203.5 102.75) (size 0.8) (layers F.Cu B.Cu) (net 21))
 (segment (start 200.66 129.54) (end 200.533 129.54) (width 0.3) (layer F.Cu) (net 12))
 (segment (start 200.533 129.54) (end 199.39 128.397) (width 0.3) (layer F.Cu) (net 12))
 (segment (start 199.39 128.397) (end 199.39 126.365) (width 0.3) (layer F.Cu) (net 12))
 (segment (start 199.39 126.365) (end 195.58 122.555) (width 0.3) (layer F.Cu) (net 12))
 (segment (start 195.58 122.555) (end 195.58 114.3) (width 0.3) (layer F.Cu) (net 12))
 (segment (start 195.58 114.3) (end 196.99 112.89) (width 0.3) (layer F.Cu) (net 12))
 (segment (start 196.99 112.89) (end 196.99 110.25) (width 0.3) (layer F.Cu) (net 12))
 (segment (start 193.04 127) (end 193.04 125.46) (width 0.3) (layer B.Cu) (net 9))
 (segment (start 193.04 125.46) (end 194 124.5) (width 0.3) (layer B.Cu) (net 9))
 (segment (start 194 124.5) (end 194 118.5) (width 0.3) (layer F.Cu) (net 9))
 (segment (start 194 118.5) (end 190.99 115.49) (width 0.3) (layer F.Cu) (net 9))
 (segment (start 190.99 115.49) (end 190.99 110.25) (width 0.3) (layer F.Cu) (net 9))
 (via (at 194 124.5) (size 0.8) (layers F.Cu B.Cu) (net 9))
 (segment (start 198.12 129.54) (end 196.85 128.27) (width 0.3) (layer F.Cu) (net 11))
 (segment (start 196.85 128.27) (end 196.85 125.73) (width 0.3) (layer F.Cu) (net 11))
 (segment (start 196.85 125.73) (end 194.945 123.825) (width 0.3) (layer F.Cu) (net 11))
 (segment (start 194.945 123.825) (end 194.945 110.295) (width 0.3) (layer F.Cu) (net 11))
 (segment (start 194.945 110.295) (end 194.99 110.25) (width 0.3) (layer F.Cu) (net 11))
 (segment (start 190.5 127) (end 190.5 119.38) (width 0.3) (layer F.Cu) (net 10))
 (segment (start 190.5 119.38) (end 185.42 114.3) (width 0.3) (layer F.Cu) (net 10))
 (segment (start 185.42 114.3) (end 185.42 109.22) (width 0.3) (layer F.Cu) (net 10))
 (segment (start 185.42 109.22) (end 186.69 107.95) (width 0.3) (layer F.Cu) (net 10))
 (segment (start 186.69 107.95) (end 191.77 107.95) (width 0.3) (layer F.Cu) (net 10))
 (segment (start 191.77 107.95) (end 192.99 109.17) (width 0.3) (layer F.Cu) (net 10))
 (segment (start 192.99 109.17) (end 192.99 110.25) (width 0.3) (layer F.Cu) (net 10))
 (segment (start 189.23 110.49) (end 188.99 110.25) (width 0.3) (layer F.Cu) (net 8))
 (segment (start 195.58 129.54) (end 194.31 128.27) (width 0.3) (layer F.Cu) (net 8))
 (segment (start 194.31 128.27) (end 194.31 126.31) (width 0.3) (layer F.Cu) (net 8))
 (segment (start 194.31 126.31) (end 192.5 124.5) (width 0.3) (layer F.Cu) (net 8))
 (segment (start 192.5 124.5) (end 192.5 119) (width 0.3) (layer F.Cu) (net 8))
 (segment (start 192.5 119) (end 188.99 115.49) (width 0.3) (layer F.Cu) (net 8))
 (segment (start 188.99 115.49) (end 188.99 110.25) (width 0.3) (layer F.Cu) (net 8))
 (segment (start 187.96 127) (end 187.96 121.285) (width 0.3) (layer B.Cu) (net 16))
 (segment (start 187.96 121.285) (end 180.5 113.825) (width 0.3) (layer B.Cu) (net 16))
 (segment (start 180.5 113.825) (end 180.5 105.5) (width 0.3) (layer B.Cu) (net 16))
 (segment (start 180.5 105.5) (end 181.5 104.5) (width 0.3) (layer B.Cu) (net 16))
 (segment (start 181.5 104.5) (end 184 104.5) (width 0.3) (layer F.Cu) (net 16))
 (via (at 181.5 104.5) (size 0.8) (layers F.Cu B.Cu) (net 16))
 (segment (start 186.69 110.55) (end 186.99 110.25) (width 0.3) (layer F.Cu) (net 7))
 (segment (start 193.04 129.54) (end 191.77 128.27) (width 0.3) (layer F.Cu) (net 7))
 (segment (start 191.77 128.27) (end 191.77 119.38) (width 0.3) (layer F.Cu) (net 7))
 (segment (start 191.77 119.38) (end 186.99 114.6) (width 0.3) (layer F.Cu) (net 7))
 (segment (start 186.99 114.6) (end 186.99 110.25) (width 0.3) (layer F.Cu) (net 7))
 (segment (start 181.5 106) (end 182.5 106) (width 0.3) (layer B.Cu) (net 17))
 (segment (start 182.5 106) (end 183 105.5) (width 0.3) (layer B.Cu) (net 17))
 (segment (start 183 105.5) (end 183 101.5) (width 0.3) (layer B.Cu) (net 17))
 (segment (start 183 101.5) (end 182.5 101) (width 0.3) (layer B.Cu) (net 17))
 (segment (start 182.5 101) (end 181 101) (width 0.3) (layer B.Cu) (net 17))
 (segment (start 181 101) (end 179 103) (width 0.3) (layer B.Cu) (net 17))
 (segment (start 179 103) (end 179 114) (width 0.3) (layer B.Cu) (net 17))
 (segment (start 179 114) (end 186 121) (width 0.3) (layer B.Cu) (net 17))
 (segment (start 186 121) (end 186 126.42) (width 0.3) (layer B.Cu) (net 17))
 (segment (start 186 126.42) (end 185.42 127) (width 0.3) (layer B.Cu) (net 17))
 (segment (start 184 106.5) (end 182 106.5) (width 0.3) (layer F.Cu) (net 17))
 (segment (start 182 106.5) (end 181.5 106) (width 0.3) (layer F.Cu) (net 17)) (via (at 181.5 106) (size 0.8) (layers F.Cu B.Cu) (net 17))
 (segment (start 181.5 102.5) (end 179.75 104.25) (width 0.3) (layer B.Cu) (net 15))
 (segment (start 179.75 104.25) (end 179.75 113.89) (width 0.3) (layer B.Cu) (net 15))
 (segment (start 179.75 113.89) (end 186.69 120.83) (width 0.3) (layer B.Cu) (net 15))
 (segment (start 186.69 120.83) (end 186.69 128.27) (width 0.3) (layer B.Cu) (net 15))
 (segment (start 186.69 128.27) (end 185.42 129.54) (width 0.3) (layer B.Cu) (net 15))
 (segment (start 184 102.5) (end 181.5 102.5) (width 0.3) (layer F.Cu) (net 15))
 (via (at 181.5 102.5) (size 0.8) (layers F.Cu B.Cu) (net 15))
 (segment (start 187.96 129.54) (end 189.23 128.27) (width 0.3) (layer B.Cu) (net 18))
 (segment (start 189.23 128.27) (end 189.23 121.285) (width 0.3) (layer B.Cu) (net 18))
 (segment (start 189.23 121.285) (end 181.61 113.665) (width 0.3) (layer B.Cu) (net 18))
 (segment (start 181.61 113.665) (end 181.61 111.76) (width 0.3) (layer B.Cu) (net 18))
 (segment (start 181.61 111.76) (end 183.515 109.855) (width 0.3) (layer B.Cu) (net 18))
 (segment (start 183.515 109.855) (end 196.215 109.855) (width 0.3) (layer B.Cu) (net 18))
 (segment (start 196.215 109.855) (end 199.57 106.5) (width 0.3) (layer B.Cu) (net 18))
 (segment (start 199.57 106.5) (end 201.9 106.5) (width 0.3) (layer B.Cu) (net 18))
 (segment (start 201.9 106.5) (end 200 106.5) (width 0.3) (layer F.Cu) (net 18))
 (via (at 201.9 106.5) (size 0.8) (layers F.Cu B.Cu) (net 18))
 (segment (start 184 98.5) (end 180.9 98.5) (width 0.3) (layer F.Cu) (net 6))
 (segment (start 180.9 98.5) (end 179.07 100.33) (width 0.3) (layer F.Cu) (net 6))
 (segment (start 179.07 100.33) (end 179.07 107.72) (width 0.3) (layer F.Cu) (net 6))
 (segment (start 179.07 107.72) (end 181 109.65) (width 0.3) (layer F.Cu) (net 6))
 (segment (start 204.85 106.2294) (end 206.5255 107.2145) (width 0.25) (layer F.Cu) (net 22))
 (segment (start 206.5255 107.2145) (end 206.7 107.389) (width 0.3) (layer F.Cu) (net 22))
 (segment (start 206.5255 107.2145) (end 206.693 107.313) (width 0.25) (layer F.Cu) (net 22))
 (segment (start 204.85 106.2294) (end 204.85 106.25) (width 0.3) (layer F.Cu) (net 22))
 (segment (start 201.1 98.5) (end 202 98.5) (width 0.3) (layer F.Cu) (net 22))
 (segment (start 202 98.5) (end 204.85 101.35) (width 0.3) (layer F.Cu) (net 22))
 (segment (start 204.85 101.35) (end 204.85 106.2294) (width 0.3) (layer F.Cu) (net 22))
 (segment (start 204.8 106.2) (end 204.85 106.2294) (width 0.25) (layer F.Cu) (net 22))
 (segment (start 200.3 98.5) (end 201.1 98.5) (width 0.3) (layer F.Cu) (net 22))
 (segment (start 200 98.5) (end 200.3 98.5) (width 0.3) (layer F.Cu) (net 22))
 (segment (start 200.3 98.5) (end 201.1 98.5) (width 0.3) (layer F.Cu) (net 22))
 (segment (start 203.99 114.66) (end 203.99 114.01) (width 0.3) (layer F.Cu) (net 22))
 (segment (start 203.99 114.01) (end 206.7 111.3) (width 0.3) (layer F.Cu) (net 22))
 (segment (start 206.7 111.3) (end 206.7 107.389) (width 0.3) (layer F.Cu) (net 22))
 (segment (start 202.5 96.5) (end 203.8 95.2) (width 0.3) (layer F.Cu) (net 23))
 (segment (start 203.8 95.2) (end 204.45 95.2) (width 0.3) (layer F.Cu) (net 23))
 (segment (start 201.1 96.5) (end 202.5 96.5) (width 0.3) (layer F.Cu) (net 23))
 (segment (start 200 96.5) (end 201.1 96.5) (width 0.3) (layer F.Cu) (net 23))
 (segment (start 200 96.5) (end 201.1 96.5) (width 0.3) (layer F.Cu) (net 23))
 (segment (start 204.45 97.8) (end 203.8 97.8) (width 0.3) (layer F.Cu) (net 23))
 (segment (start 203.8 97.8) (end 202.5 96.5) (width 0.3) (layer F.Cu) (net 23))
 (segment (start 207.56 103.4009) (end 207.56 98.21) (width 0.3) (layer F.Cu) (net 25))
 (segment (start 207.56 98.21) (end 207.15 97.8) (width 0.3) (layer F.Cu) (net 25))
 (segment (start 207.56 103.401) (end 207.56 103.4009) (width 0.3) (layer F.Cu) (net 25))
 (segment (start 207.56 103.4009) (end 207.56 98.21) (width 0.3) (layer F.Cu) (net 25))
 (segment (start 207.56 98.21) (end 207.15 97.8) (width 0.3) (layer F.Cu) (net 25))
 (segment (start 207.56 103.401) (end 207.56 103.4009) (width 0.3) (layer F.Cu) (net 25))
 (segment (start 208.25 113.65) (end 208.25 105.341) (width 0.3) (layer F.Cu) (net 25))
 (segment (start 208.25 105.341) (end 207.56 104.651) (width 0.3) (layer F.Cu) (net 25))
 (segment (start 207.56 104.651) (end 207.56 103.401) (width 0.3) (layer F.Cu) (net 25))
 (segment (start 207.75 98.4) (end 207.15 97.8) (width 0.3) (layer F.Cu) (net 25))
 (segment (start 208.25 113.65) (end 205.85 116.05) (width 0.25) (layer F.Cu) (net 25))
 (segment (start 205.85 116.05) (end 205.85 118.65) (width 0.25) (layer F.Cu) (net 25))
 (segment (start 206.29 105.6006) (end 206.29 104.99) (width 0.3) (layer F.Cu) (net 24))
 (segment (start 206.29 104.99) (end 205.75 104.45) (width 0.3) (layer F.Cu) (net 24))
 (segment (start 205.75 104.45) (end 205.75 94) (width 0.3) (layer F.Cu) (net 24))
 (segment (start 205.75 94) (end 205.25 93.5) (width 0.3) (layer F.Cu) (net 24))
 (segment (start 205.25 93.5) (end 202.5 93.5) (width 0.3) (layer F.Cu) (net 24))
 (segment (start 202.5 93.5) (end 201.5 94.5) (width 0.3) (layer F.Cu) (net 24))
 (segment (start 201.5 94.5) (end 200.8 94.5) (width 0.3) (layer F.Cu) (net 24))
 (segment (start 205.85 114.35) (end 205.9 114.35) (width 0.3) (layer F.Cu) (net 24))
 (segment (start 205.9 114.35) (end 207.5 112.75) (width 0.3) (layer F.Cu) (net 24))
 (segment (start 207.5 112.75) (end 207.5 106.811) (width 0.3) (layer F.Cu) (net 24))
 (segment (start 207.5 106.811) (end 206.29 105.601) (width 0.3) (layer F.Cu) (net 24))
 (segment (start 206.29 105.601) (end 206.29 105.6006) (width 0.3) (layer F.Cu) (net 24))
 (segment (start 200.8 94.5) (end 200 94.5) (width 0.3) (layer F.Cu) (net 24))
 (segment (start 200.8 94.5) (end 200 94.5) (width 0.3) (layer F.Cu) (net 24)))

